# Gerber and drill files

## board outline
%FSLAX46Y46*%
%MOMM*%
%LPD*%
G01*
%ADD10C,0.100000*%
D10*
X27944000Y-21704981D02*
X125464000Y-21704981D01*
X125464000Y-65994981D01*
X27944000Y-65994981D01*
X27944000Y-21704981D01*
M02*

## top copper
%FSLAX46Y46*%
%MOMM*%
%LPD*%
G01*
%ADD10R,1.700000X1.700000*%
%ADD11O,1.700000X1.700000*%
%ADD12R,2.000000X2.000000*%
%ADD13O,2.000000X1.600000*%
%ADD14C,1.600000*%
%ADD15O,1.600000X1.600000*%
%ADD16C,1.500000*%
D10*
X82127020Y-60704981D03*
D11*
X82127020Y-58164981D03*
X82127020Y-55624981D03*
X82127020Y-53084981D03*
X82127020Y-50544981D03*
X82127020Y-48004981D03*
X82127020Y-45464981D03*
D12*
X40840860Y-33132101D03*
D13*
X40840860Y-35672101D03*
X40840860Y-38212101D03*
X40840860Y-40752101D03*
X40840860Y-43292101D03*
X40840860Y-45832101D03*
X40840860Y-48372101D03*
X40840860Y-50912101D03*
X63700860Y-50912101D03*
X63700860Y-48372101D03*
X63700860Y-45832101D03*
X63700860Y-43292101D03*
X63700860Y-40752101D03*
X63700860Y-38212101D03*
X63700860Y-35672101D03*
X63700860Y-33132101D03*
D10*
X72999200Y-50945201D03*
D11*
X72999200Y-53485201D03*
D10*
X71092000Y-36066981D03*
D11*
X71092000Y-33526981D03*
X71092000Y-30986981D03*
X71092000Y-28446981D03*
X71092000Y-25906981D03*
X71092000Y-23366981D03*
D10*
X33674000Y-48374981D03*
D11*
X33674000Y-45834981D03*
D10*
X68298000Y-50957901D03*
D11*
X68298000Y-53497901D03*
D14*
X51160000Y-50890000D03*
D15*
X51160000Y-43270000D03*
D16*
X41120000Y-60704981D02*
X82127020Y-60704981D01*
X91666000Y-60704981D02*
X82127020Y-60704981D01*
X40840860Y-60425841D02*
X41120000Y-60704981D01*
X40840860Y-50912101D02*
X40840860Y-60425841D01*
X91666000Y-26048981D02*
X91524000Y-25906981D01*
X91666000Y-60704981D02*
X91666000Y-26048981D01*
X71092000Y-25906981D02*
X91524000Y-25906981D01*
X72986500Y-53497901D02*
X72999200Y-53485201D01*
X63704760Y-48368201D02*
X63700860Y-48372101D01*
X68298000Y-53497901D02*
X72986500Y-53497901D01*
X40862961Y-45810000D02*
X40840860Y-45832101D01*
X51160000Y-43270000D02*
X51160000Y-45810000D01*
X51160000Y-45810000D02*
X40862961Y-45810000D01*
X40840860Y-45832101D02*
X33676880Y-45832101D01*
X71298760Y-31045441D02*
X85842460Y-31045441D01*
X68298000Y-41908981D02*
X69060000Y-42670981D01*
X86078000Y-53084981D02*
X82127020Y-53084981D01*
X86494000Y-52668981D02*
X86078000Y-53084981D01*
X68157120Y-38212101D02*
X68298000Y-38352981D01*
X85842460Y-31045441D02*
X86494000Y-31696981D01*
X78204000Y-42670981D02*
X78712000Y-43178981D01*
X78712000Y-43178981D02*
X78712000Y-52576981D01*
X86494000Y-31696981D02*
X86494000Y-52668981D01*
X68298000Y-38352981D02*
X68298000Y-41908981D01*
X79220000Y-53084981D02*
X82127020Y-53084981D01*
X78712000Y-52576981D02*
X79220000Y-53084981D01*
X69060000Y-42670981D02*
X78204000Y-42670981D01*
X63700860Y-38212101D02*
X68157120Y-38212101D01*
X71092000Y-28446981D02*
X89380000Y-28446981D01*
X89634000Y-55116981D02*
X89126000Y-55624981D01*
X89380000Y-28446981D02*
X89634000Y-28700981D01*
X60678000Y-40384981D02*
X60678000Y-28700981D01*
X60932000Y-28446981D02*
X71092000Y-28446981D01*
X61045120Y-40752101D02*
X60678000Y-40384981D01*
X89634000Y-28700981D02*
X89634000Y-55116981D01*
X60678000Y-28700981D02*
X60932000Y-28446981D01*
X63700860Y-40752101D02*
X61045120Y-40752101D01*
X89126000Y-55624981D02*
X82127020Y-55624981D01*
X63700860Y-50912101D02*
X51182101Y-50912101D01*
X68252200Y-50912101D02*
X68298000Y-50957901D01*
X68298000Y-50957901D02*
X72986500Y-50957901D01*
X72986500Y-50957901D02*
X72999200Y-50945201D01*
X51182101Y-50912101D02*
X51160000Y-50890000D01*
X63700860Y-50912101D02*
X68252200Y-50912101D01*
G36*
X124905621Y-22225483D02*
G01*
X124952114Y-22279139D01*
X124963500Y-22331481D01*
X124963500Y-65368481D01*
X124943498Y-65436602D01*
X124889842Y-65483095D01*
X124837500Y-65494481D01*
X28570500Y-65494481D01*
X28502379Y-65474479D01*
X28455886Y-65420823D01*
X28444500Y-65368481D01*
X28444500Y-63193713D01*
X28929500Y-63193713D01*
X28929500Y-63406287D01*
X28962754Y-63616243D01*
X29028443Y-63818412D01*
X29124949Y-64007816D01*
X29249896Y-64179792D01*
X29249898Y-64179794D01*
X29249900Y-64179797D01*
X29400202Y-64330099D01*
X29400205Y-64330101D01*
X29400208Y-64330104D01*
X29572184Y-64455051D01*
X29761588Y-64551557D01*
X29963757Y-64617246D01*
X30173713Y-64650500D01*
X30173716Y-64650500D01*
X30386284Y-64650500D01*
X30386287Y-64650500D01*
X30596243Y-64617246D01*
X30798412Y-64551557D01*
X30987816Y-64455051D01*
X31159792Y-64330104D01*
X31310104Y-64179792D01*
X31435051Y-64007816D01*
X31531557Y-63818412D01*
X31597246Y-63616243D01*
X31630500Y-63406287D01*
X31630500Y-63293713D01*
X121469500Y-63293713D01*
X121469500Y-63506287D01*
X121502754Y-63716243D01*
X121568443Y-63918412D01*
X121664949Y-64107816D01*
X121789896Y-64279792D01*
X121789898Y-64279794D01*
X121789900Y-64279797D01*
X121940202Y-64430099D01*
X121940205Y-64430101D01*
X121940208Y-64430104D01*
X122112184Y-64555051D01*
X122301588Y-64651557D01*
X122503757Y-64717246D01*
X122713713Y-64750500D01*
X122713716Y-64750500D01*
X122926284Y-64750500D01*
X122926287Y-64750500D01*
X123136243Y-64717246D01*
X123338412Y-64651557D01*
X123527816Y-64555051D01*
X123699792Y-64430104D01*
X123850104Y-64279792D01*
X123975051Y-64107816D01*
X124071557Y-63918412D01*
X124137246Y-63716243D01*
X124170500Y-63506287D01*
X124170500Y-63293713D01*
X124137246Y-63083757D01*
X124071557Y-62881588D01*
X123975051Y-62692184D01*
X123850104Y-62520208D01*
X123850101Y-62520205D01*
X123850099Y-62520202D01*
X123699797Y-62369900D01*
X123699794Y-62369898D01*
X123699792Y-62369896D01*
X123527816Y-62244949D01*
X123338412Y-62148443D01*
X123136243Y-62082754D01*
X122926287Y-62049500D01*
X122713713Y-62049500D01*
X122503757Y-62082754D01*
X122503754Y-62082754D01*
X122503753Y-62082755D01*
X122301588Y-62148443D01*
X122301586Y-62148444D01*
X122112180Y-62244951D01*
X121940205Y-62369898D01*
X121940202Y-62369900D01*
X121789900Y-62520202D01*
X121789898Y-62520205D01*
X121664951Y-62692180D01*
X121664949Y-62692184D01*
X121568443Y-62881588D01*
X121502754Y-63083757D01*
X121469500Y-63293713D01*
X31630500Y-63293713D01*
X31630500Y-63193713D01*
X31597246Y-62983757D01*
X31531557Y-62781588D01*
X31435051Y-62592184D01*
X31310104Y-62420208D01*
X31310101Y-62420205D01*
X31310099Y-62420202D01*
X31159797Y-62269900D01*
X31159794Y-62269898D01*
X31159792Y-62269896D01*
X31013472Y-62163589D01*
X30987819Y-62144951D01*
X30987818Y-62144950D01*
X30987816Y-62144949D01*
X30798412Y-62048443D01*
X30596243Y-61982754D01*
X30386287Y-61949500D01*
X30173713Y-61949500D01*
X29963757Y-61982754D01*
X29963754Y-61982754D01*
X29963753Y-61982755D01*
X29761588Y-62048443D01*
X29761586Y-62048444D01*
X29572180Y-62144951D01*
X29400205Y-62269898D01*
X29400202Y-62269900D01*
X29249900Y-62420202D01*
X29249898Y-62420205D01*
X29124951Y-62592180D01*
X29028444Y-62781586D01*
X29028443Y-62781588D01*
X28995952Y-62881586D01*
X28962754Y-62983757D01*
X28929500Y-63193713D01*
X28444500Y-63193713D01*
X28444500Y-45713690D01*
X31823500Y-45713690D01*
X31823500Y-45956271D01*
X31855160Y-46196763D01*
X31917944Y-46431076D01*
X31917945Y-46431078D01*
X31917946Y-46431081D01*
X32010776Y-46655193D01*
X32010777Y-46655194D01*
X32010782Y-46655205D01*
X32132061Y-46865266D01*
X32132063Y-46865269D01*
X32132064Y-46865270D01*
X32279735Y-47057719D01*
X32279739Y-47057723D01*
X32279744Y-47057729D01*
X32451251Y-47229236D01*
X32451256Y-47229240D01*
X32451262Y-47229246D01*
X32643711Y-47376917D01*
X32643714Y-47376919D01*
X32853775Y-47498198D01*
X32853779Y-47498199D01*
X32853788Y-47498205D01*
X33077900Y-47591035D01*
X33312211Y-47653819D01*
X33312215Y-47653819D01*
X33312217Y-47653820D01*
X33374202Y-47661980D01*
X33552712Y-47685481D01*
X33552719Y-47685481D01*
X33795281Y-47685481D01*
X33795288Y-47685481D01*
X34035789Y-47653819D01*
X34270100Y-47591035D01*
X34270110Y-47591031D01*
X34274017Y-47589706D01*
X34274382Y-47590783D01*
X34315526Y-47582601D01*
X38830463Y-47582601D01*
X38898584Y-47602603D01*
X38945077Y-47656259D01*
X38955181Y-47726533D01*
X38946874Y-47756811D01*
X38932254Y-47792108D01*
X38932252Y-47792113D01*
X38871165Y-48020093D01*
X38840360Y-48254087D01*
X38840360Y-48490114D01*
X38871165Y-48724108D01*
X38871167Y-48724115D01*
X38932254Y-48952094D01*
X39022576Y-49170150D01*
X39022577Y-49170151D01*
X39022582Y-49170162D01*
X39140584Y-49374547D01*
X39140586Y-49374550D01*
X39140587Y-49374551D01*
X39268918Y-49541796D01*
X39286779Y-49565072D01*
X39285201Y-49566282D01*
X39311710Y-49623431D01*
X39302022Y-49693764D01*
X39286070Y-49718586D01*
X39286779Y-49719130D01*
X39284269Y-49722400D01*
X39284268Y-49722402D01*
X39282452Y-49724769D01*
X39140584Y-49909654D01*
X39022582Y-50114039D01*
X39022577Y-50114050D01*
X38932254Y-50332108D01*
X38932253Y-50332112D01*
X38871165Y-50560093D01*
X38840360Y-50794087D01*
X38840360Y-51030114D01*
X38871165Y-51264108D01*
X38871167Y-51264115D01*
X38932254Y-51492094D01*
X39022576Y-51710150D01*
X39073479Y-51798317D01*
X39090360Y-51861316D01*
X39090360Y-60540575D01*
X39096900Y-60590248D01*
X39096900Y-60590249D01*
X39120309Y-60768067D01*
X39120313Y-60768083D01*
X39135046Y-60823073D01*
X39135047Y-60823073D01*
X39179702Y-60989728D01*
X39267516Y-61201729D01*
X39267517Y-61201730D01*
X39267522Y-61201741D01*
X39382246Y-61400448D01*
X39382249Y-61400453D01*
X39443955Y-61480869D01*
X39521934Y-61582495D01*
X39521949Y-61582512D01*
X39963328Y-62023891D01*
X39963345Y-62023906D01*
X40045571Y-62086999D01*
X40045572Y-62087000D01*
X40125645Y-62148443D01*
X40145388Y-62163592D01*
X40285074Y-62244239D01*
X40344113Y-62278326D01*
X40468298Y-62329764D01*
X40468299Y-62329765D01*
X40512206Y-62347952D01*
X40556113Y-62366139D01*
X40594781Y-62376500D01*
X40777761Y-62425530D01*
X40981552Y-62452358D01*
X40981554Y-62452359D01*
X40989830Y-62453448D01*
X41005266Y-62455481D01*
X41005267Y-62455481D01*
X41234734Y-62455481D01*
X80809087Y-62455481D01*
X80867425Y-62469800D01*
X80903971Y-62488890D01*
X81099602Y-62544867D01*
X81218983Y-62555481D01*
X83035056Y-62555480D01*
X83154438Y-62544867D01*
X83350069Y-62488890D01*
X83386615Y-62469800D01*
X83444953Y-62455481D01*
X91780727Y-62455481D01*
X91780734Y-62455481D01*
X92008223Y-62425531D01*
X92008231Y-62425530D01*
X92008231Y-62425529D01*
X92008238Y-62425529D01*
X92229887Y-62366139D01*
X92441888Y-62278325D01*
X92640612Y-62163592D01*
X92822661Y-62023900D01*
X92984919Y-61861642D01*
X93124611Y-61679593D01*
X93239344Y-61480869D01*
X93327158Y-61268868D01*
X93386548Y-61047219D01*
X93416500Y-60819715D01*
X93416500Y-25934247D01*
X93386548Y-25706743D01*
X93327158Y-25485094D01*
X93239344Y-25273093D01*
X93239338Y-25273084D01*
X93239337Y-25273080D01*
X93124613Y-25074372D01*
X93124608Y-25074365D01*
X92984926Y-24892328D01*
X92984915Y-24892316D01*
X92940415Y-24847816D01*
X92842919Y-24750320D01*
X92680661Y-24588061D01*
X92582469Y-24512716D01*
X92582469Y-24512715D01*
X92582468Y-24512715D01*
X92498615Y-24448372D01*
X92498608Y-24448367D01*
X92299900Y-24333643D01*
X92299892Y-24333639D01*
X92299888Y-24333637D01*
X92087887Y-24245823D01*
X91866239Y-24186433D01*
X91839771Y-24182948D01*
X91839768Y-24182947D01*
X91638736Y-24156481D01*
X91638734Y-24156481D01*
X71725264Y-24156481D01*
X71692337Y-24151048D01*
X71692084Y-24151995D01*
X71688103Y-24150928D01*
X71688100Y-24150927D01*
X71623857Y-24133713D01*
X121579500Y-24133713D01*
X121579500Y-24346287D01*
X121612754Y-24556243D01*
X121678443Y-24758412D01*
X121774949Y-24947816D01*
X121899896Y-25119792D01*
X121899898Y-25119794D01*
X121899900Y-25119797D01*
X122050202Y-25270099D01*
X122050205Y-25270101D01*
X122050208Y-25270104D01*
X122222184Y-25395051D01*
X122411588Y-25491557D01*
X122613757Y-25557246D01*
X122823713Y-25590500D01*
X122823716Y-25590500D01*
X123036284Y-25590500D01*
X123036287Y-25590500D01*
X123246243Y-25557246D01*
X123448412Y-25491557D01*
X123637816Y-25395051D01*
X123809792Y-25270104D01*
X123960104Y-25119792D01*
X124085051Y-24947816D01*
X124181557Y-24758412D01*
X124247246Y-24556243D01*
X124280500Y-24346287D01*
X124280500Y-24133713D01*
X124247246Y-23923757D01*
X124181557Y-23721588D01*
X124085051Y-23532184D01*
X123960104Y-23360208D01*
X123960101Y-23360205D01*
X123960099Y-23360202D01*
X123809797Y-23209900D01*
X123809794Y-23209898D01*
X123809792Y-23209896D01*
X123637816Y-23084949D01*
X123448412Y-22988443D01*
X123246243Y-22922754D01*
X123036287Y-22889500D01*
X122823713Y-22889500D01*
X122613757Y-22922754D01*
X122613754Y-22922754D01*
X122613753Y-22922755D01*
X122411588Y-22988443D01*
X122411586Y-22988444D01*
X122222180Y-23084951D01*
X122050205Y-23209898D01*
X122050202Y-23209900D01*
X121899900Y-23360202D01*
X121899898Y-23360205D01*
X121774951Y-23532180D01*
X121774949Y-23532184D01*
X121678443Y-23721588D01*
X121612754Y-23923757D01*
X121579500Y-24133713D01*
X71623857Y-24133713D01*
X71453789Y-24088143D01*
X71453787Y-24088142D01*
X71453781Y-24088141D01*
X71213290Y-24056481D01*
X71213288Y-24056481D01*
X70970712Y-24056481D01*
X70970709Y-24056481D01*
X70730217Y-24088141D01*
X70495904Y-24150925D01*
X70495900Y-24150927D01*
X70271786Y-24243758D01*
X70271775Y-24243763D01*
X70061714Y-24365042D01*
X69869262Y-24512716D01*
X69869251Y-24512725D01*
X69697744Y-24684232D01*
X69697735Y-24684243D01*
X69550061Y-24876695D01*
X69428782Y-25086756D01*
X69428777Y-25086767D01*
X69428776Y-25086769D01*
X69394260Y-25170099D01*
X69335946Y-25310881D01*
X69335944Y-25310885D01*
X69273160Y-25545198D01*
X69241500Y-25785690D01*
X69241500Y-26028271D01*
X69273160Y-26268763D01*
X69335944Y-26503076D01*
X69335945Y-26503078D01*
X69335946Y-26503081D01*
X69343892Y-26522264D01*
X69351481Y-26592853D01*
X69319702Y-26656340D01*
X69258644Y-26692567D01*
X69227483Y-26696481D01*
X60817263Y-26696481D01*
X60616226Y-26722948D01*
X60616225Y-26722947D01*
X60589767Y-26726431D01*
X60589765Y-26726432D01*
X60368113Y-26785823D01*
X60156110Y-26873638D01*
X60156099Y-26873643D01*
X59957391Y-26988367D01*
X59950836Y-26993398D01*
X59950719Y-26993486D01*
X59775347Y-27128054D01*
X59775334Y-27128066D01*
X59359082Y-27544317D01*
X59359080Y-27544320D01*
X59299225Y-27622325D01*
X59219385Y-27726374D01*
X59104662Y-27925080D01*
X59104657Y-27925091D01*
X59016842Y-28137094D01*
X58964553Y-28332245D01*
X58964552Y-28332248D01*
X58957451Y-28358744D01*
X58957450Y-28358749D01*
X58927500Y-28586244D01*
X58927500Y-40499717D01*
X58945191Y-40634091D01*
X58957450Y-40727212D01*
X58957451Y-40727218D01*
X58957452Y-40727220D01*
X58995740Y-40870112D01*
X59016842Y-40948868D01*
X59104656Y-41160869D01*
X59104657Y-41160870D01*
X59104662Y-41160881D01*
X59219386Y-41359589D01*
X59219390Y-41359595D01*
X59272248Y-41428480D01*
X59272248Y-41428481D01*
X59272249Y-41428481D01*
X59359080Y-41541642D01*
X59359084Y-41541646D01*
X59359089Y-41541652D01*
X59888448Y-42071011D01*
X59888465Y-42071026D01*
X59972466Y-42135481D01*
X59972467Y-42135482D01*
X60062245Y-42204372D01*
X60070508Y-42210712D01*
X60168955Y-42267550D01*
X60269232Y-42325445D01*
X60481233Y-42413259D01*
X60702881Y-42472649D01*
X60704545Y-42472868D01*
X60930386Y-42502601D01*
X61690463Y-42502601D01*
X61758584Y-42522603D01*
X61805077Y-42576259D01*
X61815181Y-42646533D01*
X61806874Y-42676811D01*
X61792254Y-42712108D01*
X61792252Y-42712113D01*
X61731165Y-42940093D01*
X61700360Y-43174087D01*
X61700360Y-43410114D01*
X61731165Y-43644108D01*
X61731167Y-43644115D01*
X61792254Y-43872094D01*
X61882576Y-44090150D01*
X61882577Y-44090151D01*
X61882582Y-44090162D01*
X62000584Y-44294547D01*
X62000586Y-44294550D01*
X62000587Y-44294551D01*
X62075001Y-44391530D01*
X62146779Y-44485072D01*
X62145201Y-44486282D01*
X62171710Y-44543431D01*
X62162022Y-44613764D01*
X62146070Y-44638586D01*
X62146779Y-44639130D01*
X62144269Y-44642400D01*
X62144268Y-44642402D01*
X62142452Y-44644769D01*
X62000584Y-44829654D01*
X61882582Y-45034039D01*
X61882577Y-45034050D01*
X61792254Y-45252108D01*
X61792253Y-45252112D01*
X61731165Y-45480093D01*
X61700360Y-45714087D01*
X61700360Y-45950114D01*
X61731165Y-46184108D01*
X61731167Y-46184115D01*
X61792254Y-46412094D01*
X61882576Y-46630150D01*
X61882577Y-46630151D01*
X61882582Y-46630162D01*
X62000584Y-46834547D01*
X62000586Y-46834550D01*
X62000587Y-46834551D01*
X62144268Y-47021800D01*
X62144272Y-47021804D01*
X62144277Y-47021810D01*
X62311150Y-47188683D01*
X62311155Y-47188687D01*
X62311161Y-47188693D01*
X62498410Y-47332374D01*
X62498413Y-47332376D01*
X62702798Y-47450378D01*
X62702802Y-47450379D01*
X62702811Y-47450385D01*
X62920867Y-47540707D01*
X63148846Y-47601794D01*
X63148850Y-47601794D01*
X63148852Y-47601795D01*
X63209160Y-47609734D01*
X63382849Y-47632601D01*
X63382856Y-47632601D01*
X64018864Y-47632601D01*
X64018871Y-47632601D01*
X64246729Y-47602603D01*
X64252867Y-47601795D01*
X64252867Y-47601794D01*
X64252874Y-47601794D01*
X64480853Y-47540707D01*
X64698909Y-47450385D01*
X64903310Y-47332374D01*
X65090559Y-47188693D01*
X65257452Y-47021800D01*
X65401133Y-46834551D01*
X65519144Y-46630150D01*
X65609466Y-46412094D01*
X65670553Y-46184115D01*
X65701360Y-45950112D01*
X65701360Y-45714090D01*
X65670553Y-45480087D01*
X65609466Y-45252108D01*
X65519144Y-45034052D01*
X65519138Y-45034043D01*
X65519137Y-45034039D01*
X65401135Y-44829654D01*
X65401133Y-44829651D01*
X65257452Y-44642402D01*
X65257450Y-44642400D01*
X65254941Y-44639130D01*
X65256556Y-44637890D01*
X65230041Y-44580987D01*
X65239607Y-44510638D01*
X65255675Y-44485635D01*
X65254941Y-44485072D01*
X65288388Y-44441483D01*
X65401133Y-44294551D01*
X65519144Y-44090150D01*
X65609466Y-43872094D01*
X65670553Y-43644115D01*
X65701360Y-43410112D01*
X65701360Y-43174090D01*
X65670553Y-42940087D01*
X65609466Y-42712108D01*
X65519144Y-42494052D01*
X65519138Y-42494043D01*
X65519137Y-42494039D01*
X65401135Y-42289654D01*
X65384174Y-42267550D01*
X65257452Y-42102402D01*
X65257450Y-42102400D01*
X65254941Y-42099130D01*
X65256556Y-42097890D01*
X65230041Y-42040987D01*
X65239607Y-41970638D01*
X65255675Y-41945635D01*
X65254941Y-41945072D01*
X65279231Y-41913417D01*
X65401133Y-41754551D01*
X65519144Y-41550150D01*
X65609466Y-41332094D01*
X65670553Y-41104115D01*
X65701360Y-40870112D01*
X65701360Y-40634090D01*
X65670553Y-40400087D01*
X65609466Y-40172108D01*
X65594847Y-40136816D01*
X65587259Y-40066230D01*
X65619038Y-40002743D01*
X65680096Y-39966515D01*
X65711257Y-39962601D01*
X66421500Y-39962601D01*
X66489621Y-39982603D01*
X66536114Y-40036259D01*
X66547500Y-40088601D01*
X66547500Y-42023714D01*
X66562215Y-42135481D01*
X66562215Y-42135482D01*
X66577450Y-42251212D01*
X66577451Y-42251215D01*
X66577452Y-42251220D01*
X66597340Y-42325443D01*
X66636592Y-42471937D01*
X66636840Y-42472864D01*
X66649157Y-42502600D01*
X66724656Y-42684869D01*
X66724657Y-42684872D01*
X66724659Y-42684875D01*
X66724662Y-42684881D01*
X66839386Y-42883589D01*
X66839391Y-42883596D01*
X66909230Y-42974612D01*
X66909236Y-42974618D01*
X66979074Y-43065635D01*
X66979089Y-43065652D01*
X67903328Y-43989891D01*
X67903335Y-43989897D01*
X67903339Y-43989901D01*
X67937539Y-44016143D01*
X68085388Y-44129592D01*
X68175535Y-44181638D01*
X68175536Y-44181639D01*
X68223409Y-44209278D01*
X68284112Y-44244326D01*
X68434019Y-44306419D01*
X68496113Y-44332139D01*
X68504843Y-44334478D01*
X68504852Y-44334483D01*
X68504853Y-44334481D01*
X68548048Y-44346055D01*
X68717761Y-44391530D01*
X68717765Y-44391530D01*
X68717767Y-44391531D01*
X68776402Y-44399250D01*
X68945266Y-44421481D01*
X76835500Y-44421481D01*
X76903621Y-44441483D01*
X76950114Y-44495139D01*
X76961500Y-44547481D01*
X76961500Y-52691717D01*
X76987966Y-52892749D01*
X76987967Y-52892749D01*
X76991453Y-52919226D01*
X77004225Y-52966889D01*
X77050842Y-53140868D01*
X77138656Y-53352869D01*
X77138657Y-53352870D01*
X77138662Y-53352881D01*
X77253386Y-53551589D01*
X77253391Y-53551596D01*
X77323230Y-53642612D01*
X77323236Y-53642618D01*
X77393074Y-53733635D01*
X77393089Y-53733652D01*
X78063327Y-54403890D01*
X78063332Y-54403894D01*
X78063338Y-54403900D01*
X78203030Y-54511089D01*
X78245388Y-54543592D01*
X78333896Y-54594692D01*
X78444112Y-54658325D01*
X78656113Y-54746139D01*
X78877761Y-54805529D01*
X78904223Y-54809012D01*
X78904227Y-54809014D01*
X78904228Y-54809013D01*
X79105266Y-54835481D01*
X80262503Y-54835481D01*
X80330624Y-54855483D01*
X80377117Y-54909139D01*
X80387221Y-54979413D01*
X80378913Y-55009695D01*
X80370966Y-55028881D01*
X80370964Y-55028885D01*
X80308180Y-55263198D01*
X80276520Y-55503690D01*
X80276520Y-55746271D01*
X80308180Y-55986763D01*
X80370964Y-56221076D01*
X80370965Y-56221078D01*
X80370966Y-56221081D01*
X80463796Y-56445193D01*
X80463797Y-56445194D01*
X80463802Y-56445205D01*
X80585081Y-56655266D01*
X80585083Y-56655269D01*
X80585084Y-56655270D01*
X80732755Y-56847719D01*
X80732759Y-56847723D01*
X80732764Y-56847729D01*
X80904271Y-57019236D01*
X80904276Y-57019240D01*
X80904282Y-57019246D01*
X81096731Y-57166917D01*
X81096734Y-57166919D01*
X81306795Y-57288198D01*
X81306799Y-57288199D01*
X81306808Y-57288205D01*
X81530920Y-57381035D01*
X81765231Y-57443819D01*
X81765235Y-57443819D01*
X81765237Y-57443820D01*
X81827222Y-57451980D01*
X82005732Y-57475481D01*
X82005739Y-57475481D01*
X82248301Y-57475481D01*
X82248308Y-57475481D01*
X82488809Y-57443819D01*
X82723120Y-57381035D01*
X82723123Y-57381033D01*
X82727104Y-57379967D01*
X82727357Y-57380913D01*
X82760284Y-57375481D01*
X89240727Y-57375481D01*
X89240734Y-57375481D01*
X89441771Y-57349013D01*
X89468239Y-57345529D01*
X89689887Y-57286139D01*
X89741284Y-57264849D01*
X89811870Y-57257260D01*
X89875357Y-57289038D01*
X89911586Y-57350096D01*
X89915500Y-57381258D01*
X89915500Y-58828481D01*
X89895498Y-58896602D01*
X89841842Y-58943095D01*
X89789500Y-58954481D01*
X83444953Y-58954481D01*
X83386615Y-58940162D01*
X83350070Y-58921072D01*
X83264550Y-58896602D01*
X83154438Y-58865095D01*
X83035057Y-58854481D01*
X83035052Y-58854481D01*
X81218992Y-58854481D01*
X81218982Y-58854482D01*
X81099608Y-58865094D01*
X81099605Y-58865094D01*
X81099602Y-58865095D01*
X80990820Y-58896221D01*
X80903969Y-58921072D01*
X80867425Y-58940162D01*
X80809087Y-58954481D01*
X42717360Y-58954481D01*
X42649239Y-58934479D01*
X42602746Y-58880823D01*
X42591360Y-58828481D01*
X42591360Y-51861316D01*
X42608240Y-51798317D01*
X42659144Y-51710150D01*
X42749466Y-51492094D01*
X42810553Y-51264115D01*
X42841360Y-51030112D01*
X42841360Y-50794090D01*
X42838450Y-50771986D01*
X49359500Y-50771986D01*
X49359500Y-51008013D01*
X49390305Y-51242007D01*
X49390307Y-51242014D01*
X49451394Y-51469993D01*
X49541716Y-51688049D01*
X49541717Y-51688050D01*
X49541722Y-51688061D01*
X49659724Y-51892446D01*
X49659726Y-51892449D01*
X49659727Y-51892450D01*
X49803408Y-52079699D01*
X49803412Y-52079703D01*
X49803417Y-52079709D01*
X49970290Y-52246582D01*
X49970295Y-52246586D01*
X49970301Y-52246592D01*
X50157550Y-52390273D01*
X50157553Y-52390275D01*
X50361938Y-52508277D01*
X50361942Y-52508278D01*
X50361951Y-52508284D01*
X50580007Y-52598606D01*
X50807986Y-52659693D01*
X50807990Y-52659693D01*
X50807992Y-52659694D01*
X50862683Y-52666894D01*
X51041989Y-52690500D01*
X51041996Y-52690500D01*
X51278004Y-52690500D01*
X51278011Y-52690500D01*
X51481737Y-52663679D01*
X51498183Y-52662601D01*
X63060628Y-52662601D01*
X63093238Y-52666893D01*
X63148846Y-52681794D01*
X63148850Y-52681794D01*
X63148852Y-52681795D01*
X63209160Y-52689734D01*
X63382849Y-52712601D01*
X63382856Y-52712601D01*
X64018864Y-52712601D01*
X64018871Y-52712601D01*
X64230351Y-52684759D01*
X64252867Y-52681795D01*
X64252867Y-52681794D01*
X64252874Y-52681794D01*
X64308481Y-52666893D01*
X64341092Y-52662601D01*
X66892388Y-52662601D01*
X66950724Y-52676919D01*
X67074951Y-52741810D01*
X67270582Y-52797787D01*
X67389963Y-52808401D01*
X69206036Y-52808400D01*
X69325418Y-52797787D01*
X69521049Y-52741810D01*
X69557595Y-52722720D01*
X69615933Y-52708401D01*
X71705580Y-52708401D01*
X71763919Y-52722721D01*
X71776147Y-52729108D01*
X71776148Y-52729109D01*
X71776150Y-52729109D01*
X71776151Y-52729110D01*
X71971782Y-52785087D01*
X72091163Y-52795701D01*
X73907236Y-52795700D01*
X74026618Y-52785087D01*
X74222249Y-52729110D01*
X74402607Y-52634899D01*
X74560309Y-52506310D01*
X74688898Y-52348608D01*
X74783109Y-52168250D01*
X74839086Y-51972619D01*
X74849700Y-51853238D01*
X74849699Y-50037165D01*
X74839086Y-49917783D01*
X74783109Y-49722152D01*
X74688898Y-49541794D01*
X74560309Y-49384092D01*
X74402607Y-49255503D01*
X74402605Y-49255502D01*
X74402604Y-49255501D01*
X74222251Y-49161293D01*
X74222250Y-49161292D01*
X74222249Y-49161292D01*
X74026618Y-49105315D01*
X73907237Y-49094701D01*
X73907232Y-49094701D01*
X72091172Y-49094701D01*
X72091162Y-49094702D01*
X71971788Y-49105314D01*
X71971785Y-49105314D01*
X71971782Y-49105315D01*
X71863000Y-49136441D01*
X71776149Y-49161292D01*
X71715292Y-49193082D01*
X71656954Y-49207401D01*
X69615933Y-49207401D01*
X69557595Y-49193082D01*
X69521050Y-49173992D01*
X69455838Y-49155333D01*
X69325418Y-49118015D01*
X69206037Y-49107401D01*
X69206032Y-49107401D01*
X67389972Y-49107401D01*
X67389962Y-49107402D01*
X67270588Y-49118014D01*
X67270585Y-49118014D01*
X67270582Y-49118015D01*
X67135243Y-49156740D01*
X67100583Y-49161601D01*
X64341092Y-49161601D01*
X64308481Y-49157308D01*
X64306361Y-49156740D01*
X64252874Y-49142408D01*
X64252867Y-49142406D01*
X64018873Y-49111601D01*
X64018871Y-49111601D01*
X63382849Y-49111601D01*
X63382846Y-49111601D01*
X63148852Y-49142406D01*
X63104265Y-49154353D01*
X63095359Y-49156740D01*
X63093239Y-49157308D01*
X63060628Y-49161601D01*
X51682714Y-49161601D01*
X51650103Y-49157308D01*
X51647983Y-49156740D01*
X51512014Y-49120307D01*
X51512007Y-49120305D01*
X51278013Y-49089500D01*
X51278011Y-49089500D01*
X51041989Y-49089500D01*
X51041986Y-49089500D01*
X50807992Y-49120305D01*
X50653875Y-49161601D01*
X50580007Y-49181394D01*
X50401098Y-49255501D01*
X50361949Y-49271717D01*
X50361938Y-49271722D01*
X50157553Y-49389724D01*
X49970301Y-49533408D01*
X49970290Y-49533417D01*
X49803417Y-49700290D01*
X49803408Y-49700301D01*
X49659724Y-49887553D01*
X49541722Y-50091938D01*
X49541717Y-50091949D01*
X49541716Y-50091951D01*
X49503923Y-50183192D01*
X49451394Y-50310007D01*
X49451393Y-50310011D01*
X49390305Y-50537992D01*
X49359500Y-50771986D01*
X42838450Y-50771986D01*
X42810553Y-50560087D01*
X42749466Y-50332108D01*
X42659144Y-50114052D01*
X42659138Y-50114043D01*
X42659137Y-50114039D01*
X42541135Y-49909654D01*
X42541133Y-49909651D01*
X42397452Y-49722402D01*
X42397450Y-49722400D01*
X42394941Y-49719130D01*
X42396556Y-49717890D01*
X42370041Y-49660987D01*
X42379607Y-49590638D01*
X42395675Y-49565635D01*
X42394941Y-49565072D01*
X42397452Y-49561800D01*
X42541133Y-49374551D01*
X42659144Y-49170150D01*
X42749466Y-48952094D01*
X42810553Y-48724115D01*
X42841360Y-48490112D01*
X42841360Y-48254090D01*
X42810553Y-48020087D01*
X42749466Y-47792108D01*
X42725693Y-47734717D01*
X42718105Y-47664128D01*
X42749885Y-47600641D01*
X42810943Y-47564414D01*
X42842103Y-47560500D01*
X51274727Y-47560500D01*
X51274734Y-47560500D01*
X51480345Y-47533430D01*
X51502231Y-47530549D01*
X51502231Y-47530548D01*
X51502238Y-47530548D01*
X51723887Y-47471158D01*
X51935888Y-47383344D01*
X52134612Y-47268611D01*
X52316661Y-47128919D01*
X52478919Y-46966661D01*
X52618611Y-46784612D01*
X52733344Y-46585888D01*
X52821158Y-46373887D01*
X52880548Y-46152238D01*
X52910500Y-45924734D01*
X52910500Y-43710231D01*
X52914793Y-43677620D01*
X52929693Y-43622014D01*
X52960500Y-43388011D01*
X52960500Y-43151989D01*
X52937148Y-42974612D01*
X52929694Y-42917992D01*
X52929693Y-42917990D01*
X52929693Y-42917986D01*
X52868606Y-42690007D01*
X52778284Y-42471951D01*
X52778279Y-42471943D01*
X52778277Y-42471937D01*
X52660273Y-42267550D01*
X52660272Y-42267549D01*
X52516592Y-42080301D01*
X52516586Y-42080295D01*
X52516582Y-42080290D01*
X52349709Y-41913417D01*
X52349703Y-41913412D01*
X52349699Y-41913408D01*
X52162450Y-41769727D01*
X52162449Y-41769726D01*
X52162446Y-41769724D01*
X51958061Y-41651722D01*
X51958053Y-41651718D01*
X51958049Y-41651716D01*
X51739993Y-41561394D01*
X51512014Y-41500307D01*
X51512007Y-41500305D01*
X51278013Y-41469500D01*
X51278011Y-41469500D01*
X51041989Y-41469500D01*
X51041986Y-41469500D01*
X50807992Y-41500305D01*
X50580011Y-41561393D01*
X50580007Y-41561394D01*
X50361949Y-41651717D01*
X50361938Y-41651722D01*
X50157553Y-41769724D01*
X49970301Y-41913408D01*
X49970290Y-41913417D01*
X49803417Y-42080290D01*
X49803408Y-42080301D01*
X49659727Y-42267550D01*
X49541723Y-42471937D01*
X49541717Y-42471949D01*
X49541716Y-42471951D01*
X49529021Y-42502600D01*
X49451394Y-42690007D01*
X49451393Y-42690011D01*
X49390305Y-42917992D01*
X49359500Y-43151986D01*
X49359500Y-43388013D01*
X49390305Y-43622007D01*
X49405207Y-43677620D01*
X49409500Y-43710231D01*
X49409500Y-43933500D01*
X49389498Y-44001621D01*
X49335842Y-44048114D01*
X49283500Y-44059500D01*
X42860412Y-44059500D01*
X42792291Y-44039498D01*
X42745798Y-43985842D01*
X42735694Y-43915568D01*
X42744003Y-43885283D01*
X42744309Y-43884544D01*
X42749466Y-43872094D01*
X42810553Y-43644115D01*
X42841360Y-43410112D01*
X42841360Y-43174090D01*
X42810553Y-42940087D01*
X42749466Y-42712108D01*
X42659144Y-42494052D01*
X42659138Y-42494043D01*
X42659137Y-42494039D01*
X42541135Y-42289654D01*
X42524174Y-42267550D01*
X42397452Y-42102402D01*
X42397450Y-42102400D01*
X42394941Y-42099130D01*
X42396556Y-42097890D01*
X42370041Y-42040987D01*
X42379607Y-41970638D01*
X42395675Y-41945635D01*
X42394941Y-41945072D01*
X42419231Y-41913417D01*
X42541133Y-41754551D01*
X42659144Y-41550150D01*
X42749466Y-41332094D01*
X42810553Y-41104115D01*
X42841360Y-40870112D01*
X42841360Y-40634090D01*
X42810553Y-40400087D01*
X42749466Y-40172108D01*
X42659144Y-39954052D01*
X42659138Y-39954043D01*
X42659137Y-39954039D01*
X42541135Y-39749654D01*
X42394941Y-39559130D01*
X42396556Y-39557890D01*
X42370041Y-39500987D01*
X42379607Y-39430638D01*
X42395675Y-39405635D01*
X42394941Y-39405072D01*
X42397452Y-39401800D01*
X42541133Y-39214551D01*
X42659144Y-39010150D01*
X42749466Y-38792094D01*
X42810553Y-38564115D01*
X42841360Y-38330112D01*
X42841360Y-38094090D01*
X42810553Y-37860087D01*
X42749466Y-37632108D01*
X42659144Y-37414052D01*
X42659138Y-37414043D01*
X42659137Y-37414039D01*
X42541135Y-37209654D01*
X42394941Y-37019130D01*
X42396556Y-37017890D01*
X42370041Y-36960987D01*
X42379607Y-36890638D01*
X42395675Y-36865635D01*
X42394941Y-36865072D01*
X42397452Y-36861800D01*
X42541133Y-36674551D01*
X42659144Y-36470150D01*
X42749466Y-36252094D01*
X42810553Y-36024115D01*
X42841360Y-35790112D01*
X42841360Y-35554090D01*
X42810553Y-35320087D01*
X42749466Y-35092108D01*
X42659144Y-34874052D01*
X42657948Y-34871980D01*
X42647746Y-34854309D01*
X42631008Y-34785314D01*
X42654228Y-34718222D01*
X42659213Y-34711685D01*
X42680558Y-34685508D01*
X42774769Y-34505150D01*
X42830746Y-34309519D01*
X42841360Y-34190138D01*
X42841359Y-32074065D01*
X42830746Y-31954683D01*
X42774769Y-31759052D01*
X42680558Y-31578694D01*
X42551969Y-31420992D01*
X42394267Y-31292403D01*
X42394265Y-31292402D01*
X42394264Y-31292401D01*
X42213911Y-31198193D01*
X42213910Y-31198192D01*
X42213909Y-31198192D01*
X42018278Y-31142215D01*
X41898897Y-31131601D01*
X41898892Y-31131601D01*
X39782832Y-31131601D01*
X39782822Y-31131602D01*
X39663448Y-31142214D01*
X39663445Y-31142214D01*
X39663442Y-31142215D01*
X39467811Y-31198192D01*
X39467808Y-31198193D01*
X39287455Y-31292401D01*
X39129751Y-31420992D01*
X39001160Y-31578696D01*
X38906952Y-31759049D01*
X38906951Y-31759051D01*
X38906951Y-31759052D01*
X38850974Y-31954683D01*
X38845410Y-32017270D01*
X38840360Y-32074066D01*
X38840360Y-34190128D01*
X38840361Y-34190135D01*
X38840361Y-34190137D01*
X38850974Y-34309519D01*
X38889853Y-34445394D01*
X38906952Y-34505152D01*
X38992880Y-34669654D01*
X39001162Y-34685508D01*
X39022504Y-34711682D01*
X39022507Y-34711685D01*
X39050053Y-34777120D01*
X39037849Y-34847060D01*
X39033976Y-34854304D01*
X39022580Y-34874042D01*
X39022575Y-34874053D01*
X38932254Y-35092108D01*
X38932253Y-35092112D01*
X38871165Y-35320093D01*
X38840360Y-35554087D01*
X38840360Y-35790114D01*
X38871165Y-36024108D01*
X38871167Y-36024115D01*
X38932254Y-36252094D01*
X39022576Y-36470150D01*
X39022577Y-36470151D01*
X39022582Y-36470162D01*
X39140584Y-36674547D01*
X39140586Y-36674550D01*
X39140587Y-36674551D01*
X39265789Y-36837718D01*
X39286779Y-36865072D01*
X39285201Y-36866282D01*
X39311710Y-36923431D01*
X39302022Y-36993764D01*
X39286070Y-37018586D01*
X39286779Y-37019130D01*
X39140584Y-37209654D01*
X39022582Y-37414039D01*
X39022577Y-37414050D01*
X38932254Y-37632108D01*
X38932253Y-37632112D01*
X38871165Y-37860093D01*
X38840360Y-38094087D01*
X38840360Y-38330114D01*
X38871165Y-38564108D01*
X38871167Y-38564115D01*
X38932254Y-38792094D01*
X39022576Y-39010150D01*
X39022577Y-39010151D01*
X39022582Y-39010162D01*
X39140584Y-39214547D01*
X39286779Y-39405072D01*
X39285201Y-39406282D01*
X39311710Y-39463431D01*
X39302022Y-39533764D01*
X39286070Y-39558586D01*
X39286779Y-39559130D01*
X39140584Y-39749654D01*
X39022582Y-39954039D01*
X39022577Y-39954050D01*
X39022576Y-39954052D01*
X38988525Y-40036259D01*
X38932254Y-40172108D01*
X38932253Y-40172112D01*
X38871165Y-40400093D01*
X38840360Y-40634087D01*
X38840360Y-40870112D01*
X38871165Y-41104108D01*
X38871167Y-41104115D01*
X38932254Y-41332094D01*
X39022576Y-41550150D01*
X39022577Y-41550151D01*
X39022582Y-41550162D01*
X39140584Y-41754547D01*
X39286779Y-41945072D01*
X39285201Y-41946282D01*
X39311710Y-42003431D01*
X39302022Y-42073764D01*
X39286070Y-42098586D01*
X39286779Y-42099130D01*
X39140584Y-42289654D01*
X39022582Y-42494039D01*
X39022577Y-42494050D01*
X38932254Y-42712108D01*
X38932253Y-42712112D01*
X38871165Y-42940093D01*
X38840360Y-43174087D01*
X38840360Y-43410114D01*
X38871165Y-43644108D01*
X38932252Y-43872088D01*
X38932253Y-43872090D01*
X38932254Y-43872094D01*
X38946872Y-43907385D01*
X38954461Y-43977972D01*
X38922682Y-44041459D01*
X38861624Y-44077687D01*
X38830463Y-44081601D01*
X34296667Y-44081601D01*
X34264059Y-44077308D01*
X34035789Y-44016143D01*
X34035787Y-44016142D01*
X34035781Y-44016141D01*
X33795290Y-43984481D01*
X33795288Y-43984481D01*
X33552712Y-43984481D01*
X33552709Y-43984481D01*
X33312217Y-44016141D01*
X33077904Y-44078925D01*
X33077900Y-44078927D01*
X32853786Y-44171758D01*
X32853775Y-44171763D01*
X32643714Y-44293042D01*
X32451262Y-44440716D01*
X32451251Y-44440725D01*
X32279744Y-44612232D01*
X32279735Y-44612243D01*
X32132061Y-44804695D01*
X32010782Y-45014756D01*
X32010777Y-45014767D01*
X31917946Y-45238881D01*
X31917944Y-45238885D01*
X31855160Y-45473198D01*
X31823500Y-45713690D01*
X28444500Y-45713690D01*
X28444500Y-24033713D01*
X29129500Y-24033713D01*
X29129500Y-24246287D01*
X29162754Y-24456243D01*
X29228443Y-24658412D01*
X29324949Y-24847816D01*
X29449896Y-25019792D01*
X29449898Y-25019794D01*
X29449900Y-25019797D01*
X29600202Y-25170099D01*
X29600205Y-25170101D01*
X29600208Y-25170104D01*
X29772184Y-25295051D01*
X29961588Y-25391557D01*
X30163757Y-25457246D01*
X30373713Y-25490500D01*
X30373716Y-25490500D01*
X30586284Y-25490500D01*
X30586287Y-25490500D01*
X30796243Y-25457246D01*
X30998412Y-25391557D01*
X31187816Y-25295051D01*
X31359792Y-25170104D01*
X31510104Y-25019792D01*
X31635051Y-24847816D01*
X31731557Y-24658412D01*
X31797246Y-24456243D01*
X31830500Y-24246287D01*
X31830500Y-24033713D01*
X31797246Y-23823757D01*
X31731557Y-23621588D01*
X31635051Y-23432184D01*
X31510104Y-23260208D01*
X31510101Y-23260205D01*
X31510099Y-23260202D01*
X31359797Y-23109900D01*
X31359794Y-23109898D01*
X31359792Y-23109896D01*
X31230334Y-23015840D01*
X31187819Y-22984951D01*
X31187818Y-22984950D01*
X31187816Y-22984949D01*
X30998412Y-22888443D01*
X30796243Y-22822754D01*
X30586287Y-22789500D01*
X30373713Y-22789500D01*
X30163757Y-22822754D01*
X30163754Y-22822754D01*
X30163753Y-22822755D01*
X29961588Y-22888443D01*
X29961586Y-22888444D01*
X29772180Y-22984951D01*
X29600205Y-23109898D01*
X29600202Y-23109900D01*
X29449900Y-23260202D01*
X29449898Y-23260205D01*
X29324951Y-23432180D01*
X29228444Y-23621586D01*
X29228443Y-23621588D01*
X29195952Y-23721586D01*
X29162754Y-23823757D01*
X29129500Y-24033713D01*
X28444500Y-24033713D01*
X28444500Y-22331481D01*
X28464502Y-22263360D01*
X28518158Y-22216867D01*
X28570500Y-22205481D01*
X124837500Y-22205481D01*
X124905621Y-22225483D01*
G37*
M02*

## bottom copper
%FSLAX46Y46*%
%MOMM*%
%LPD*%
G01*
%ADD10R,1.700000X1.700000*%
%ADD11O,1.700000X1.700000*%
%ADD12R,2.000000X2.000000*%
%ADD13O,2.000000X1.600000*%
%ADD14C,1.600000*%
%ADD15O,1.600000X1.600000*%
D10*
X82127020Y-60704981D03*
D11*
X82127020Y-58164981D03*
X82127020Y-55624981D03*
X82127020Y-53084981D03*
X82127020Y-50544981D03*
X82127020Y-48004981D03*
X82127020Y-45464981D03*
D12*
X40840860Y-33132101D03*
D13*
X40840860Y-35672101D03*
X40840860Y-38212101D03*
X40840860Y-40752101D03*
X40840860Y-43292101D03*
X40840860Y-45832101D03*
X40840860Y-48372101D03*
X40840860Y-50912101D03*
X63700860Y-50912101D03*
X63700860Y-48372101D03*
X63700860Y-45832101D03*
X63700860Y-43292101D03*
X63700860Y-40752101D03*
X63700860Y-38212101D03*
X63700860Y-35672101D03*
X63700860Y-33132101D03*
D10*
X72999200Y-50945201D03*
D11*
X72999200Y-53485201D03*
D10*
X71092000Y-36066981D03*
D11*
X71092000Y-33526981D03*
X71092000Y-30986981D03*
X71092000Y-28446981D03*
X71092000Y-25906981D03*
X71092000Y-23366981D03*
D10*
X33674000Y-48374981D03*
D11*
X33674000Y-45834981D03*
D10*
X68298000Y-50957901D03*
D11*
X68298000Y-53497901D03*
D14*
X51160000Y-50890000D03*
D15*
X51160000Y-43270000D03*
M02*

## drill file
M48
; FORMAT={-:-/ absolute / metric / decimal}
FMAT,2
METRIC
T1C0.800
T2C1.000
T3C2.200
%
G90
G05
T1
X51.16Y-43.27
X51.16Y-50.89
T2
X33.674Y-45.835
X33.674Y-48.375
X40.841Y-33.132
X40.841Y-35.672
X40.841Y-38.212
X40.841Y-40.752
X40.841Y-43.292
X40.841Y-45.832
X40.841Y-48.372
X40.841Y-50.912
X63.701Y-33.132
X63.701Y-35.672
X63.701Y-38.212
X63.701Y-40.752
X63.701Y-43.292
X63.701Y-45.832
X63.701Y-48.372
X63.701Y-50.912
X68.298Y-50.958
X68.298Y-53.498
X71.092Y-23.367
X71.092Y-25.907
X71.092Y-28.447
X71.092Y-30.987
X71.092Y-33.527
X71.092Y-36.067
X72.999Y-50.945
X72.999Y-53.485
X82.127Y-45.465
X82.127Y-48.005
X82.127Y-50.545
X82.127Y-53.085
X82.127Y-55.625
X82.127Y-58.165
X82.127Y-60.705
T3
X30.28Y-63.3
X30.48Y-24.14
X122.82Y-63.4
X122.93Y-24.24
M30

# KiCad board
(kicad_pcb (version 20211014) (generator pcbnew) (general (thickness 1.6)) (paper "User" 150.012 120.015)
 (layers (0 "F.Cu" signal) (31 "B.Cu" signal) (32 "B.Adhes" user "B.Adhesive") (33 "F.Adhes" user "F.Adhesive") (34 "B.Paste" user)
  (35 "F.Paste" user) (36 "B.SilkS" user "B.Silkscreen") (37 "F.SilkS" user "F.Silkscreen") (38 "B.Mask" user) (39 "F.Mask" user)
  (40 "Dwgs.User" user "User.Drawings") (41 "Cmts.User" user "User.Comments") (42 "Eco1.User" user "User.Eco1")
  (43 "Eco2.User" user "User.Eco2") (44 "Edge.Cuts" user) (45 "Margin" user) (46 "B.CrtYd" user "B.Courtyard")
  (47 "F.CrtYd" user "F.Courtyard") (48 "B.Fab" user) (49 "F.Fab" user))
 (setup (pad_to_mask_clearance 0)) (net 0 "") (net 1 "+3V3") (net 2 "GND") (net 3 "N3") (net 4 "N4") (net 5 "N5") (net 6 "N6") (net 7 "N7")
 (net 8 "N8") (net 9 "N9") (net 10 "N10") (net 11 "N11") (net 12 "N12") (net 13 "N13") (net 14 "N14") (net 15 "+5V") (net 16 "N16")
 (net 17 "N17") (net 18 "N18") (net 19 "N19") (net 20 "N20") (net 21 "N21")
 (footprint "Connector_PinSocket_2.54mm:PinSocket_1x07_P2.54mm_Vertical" (layer "F.Cu") (at 82.12702 60.704981 180)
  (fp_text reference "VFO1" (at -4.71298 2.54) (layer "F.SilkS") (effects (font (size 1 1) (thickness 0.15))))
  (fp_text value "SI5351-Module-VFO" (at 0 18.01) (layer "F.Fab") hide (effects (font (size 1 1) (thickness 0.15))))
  (pad "1" thru_hole rect locked (at 0 0 180) (size 1.7 1.7) (drill 1) (layers *.Cu *.Mask) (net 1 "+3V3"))
  (pad "2" thru_hole oval locked (at 0 2.54 180) (size 1.7 1.7) (drill 1) (layers *.Cu *.Mask) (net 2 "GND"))
  (pad "3" thru_hole oval locked (at 0 5.08 180) (size 1.7 1.7) (drill 1) (layers *.Cu *.Mask) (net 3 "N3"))
  (pad "4" thru_hole oval locked (at 0 7.62 180) (size 1.7 1.7) (drill 1) (layers *.Cu *.Mask) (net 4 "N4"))
  (pad "5" thru_hole oval locked (at 0 10.16 180) (size 1.7 1.7) (drill 1) (layers *.Cu *.Mask) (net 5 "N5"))
  (pad "6" thru_hole oval locked (at 0 12.7 180) (size 1.7 1.7) (drill 1) (layers *.Cu *.Mask) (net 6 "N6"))
  (pad "7" thru_hole oval locked (at 0 15.24 180) (size 1.7 1.7) (drill 1) (layers *.Cu *.Mask) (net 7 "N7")))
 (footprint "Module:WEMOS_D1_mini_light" (layer "F.Cu") (at 40.84086 33.132101)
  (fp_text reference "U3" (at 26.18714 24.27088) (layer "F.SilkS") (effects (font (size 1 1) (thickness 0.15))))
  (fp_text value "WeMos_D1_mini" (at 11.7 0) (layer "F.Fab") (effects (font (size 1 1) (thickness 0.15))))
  (pad "1" thru_hole rect (at 0 0) (size 2 2) (drill 1) (layers *.Cu *.Mask) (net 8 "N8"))
  (pad "2" thru_hole oval (at 0 2.54) (size 2 1.6) (drill 1) (layers *.Cu *.Mask) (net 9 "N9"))
  (pad "3" thru_hole oval (at 0 5.08) (size 2 1.6) (drill 1) (layers *.Cu *.Mask) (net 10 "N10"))
  (pad "4" thru_hole oval (at 0 7.62) (size 2 1.6) (drill 1) (layers *.Cu *.Mask) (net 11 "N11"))
  (pad "5" thru_hole oval (at 0 10.16) (size 2 1.6) (drill 1) (layers *.Cu *.Mask) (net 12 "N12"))
  (pad "6" thru_hole oval (at 0 12.7) (size 2 1.6) (drill 1) (layers *.Cu *.Mask) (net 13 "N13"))
  (pad "7" thru_hole oval (at 0 15.24) (size 2 1.6) (drill 1) (layers *.Cu *.Mask) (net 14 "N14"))
  (pad "8" thru_hole oval (at 0 17.78) (size 2 1.6) (drill 1) (layers *.Cu *.Mask) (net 1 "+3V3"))
  (pad "9" thru_hole oval (at 22.86 17.78) (size 2 1.6) (drill 1) (layers *.Cu *.Mask) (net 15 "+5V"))
  (pad "10" thru_hole oval (at 22.86 15.24) (size 2 1.6) (drill 1) (layers *.Cu *.Mask) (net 2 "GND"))
  (pad "11" thru_hole oval (at 22.86 12.7) (size 2 1.6) (drill 1) (layers *.Cu *.Mask) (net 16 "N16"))
  (pad "12" thru_hole oval (at 22.86 10.16) (size 2 1.6) (drill 1) (layers *.Cu *.Mask) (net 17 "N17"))
  (pad "13" thru_hole oval (at 22.86 7.62) (size 2 1.6) (drill 1) (layers *.Cu *.Mask) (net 3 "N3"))
  (pad "14" thru_hole oval (at 22.86 5.08) (size 2 1.6) (drill 1) (layers *.Cu *.Mask) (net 4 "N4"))
  (pad "15" thru_hole oval (at 22.86 2.54) (size 2 1.6) (drill 1) (layers *.Cu *.Mask) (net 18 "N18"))
  (pad "16" thru_hole oval (at 22.86 0) (size 2 1.6) (drill 1) (layers *.Cu *.Mask) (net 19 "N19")))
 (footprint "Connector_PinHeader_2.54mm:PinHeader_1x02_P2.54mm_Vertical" (layer "F.Cu") (at 72.9992 50.945201)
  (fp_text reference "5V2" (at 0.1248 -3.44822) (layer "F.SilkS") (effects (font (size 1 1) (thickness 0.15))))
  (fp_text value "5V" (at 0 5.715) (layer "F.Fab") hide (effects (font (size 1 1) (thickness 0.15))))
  (pad "1" thru_hole rect locked (at 0 0) (size 1.7 1.7) (drill 1) (layers *.Cu *.Mask) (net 15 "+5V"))
  (pad "2" thru_hole oval locked (at 0 2.54) (size 1.7 1.7) (drill 1) (layers *.Cu *.Mask) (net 2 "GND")))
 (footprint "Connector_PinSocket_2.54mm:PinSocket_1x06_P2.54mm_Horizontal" (layer "F.Cu") (at 71.092 36.066981 180)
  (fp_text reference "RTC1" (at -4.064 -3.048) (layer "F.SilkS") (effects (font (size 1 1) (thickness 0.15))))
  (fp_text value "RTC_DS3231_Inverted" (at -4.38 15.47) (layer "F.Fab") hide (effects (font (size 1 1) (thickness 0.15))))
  (pad "1" thru_hole rect locked (at 0 0 180) (size 1.7 1.7) (drill 1) (layers *.Cu *.Mask) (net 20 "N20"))
  (pad "2" thru_hole oval locked (at 0 2.54 180) (size 1.7 1.7) (drill 1) (layers *.Cu *.Mask) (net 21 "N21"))
  (pad "3" thru_hole oval locked (at 0 5.08 180) (size 1.7 1.7) (drill 1) (layers *.Cu *.Mask) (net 4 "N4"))
  (pad "4" thru_hole oval locked (at 0 7.62 180) (size 1.7 1.7) (drill 1) (layers *.Cu *.Mask) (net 3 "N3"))
  (pad "5" thru_hole oval locked (at 0 10.16 180) (size 1.7 1.7) (drill 1) (layers *.Cu *.Mask) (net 1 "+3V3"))
  (pad "6" thru_hole oval locked (at 0 12.7 180) (size 1.7 1.7) (drill 1) (layers *.Cu *.Mask) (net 2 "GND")))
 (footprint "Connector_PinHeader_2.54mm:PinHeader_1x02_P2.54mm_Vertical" (layer "F.Cu") (at 33.674 48.374981 180)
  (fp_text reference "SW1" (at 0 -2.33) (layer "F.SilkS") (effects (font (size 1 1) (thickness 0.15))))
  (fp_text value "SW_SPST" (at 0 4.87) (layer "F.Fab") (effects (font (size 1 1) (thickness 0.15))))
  (pad "1" thru_hole rect locked (at 0 0 180) (size 1.7 1.7) (drill 1) (layers *.Cu *.Mask) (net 2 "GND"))
  (pad "2" thru_hole oval locked (at 0 2.54 180) (size 1.7 1.7) (drill 1) (layers *.Cu *.Mask) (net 13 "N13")))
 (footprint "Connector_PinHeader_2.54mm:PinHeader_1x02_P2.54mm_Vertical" (layer "F.Cu") (at 68.298 50.957901)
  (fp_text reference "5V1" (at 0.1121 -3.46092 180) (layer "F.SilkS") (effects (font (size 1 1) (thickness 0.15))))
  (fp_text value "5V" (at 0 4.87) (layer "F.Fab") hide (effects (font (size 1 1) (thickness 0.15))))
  (pad "1" thru_hole rect locked (at 0 0) (size 1.7 1.7) (drill 1) (layers *.Cu *.Mask) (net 15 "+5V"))
  (pad "2" thru_hole oval locked (at 0 2.54) (size 1.7 1.7) (drill 1) (layers *.Cu *.Mask) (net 2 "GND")))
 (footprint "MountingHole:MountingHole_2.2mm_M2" (layer "F.Cu") (at 122.93 24.24)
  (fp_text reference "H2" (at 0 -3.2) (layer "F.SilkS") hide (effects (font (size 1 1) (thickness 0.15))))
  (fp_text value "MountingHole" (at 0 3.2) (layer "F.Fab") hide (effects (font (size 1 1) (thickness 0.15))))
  (pad "" np_thru_hole circle (at 0 0) (size 2.2 2.2) (drill 2.2) (layers *.Cu *.Mask)))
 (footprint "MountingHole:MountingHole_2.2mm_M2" (layer "F.Cu") (at 30.28 63.3)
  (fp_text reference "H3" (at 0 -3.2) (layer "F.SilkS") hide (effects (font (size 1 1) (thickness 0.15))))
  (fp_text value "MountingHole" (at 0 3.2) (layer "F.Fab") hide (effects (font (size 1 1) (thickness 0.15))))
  (pad "" np_thru_hole circle (at 0 0) (size 2.2 2.2) (drill 2.2) (layers *.Cu *.Mask)))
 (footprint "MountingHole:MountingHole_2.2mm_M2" (layer "F.Cu") (at 30.48 24.14)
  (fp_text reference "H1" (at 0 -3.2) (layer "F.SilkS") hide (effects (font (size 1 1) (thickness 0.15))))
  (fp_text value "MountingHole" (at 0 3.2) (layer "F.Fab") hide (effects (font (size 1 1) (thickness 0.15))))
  (pad "" np_thru_hole circle (at 0 0) (size 2.2 2.2) (drill 2.2) (layers *.Cu *.Mask)))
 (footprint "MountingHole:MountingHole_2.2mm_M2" (layer "F.Cu") (at 122.82 63.4)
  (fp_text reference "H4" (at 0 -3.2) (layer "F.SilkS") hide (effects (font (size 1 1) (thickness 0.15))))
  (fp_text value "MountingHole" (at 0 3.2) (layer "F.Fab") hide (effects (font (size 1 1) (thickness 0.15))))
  (pad "" np_thru_hole circle (at 0 0) (size 2.2 2.2) (drill 2.2) (layers *.Cu *.Mask)))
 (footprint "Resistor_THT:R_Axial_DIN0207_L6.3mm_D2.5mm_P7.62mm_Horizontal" (layer "B.Cu") (at 51.16 50.89 90)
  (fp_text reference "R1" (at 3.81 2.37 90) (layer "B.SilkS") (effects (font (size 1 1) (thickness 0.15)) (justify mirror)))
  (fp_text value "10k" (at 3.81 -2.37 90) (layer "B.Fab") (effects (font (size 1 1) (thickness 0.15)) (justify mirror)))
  (pad "1" thru_hole circle (at 0 0 90) (size 1.6 1.6) (drill 0.8) (layers *.Cu *.Mask) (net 15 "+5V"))
  (pad "2" thru_hole oval (at 7.62 0 90) (size 1.6 1.6) (drill 0.8) (layers *.Cu *.Mask) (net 13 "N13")))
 (gr_rect (start 27.944 21.704981) (end 125.464 65.994981) (layer "Edge.Cuts") (width 0.1) (fill none))
 (segment (start 41.12 60.704981) (end 82.12702 60.704981) (width 1.5) (layer "F.Cu") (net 1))
 (segment (start 91.666 60.704981) (end 82.12702 60.704981) (width 1.5) (layer "F.Cu") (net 1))
 (segment (start 40.84086 60.425841) (end 41.12 60.704981) (width 1.5) (layer "F.Cu") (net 1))
 (segment (start 40.84086 50.912101) (end 40.84086 60.425841) (width 1.5) (layer "F.Cu") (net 1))
 (segment (start 91.666 26.048981) (end 91.524 25.906981) (width 1.5) (layer "F.Cu") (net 1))
 (segment (start 91.666 60.704981) (end 91.666 26.048981) (width 1.5) (layer "F.Cu") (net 1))
 (segment (start 71.092 25.906981) (end 91.524 25.906981) (width 1.5) (layer "F.Cu") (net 1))
 (segment (start 72.9865 53.497901) (end 72.9992 53.485201) (width 1.5) (layer "F.Cu") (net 2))
 (segment (start 63.70476 48.368201) (end 63.70086 48.372101) (width 1.5) (layer "F.Cu") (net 2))
 (segment (start 68.298 53.497901) (end 72.9865 53.497901) (width 1.5) (layer "F.Cu") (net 2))
 (segment (start 40.862961 45.81) (end 40.84086 45.832101) (width 1.5) (layer "F.Cu") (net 13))
 (segment (start 51.16 43.27) (end 51.16 45.81) (width 1.5) (layer "F.Cu") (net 13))
 (segment (start 51.16 45.81) (end 40.862961 45.81) (width 1.5) (layer "F.Cu") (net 13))
 (segment (start 40.84086 45.832101) (end 33.67688 45.832101) (width 1.5) (layer "F.Cu") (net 13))
 (segment (start 71.29876 31.045441) (end 85.84246 31.045441) (width 1.5) (layer "F.Cu") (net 4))
 (segment (start 68.298 41.908981) (end 69.06 42.670981) (width 1.5) (layer "F.Cu") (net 4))
 (segment (start 86.078 53.084981) (end 82.12702 53.084981) (width 1.5) (layer "F.Cu") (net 4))
 (segment (start 86.494 52.668981) (end 86.078 53.084981) (width 1.5) (layer "F.Cu") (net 4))
 (segment (start 68.15712 38.212101) (end 68.298 38.352981) (width 1.5) (layer "F.Cu") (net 4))
 (segment (start 85.84246 31.045441) (end 86.494 31.696981) (width 1.5) (layer "F.Cu") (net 4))
 (segment (start 78.204 42.670981) (end 78.712 43.178981) (width 1.5) (layer "F.Cu") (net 4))
 (segment (start 78.712 43.178981) (end 78.712 52.576981) (width 1.5) (layer "F.Cu") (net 4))
 (segment (start 86.494 31.696981) (end 86.494 52.668981) (width 1.5) (layer "F.Cu") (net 4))
 (segment (start 68.298 38.352981) (end 68.298 41.908981) (width 1.5) (layer "F.Cu") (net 4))
 (segment (start 79.22 53.084981) (end 82.12702 53.084981) (width 1.5) (layer "F.Cu") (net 4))
 (segment (start 78.712 52.576981) (end 79.22 53.084981) (width 1.5) (layer "F.Cu") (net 4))
 (segment (start 69.06 42.670981) (end 78.204 42.670981) (width 1.5) (layer "F.Cu") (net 4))
 (segment (start 63.70086 38.212101) (end 68.15712 38.212101) (width 1.5) (layer "F.Cu") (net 4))
 (segment (start 71.092 28.446981) (end 89.38 28.446981) (width 1.5) (layer "F.Cu") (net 3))
 (segment (start 89.634 55.116981) (end 89.126 55.624981) (width 1.5) (layer "F.Cu") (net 3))
 (segment (start 89.38 28.446981) (end 89.634 28.700981) (width 1.5) (layer "F.Cu") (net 3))
 (segment (start 60.678 40.384981) (end 60.678 28.700981) (width 1.5) (layer "F.Cu") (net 3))
 (segment (start 60.932 28.446981) (end 71.092 28.446981) (width 1.5) (layer "F.Cu") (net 3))
 (segment (start 61.04512 40.752101) (end 60.678 40.384981) (width 1.5) (layer "F.Cu") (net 3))
 (segment (start 89.634 28.700981) (end 89.634 55.116981) (width 1.5) (layer "F.Cu") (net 3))
 (segment (start 60.678 28.700981) (end 60.932 28.446981) (width 1.5) (layer "F.Cu") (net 3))
 (segment (start 63.70086 40.752101) (end 61.04512 40.752101) (width 1.5) (layer "F.Cu") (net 3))
 (segment (start 89.126 55.624981) (end 82.12702 55.624981) (width 1.5) (layer "F.Cu") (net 3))
 (segment (start 63.70086 50.912101) (end 51.182101 50.912101) (width 1.5) (layer "F.Cu") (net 15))
 (segment (start 68.2522 50.912101) (end 68.298 50.957901) (width 1.5) (layer "F.Cu") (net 15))
 (segment (start 68.298 50.957901) (end 72.9865 50.957901) (width 1.5) (layer "F.Cu") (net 15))
 (segment (start 72.9865 50.957901) (end 72.9992 50.945201) (width 1.5) (layer "F.Cu") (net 15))
 (segment (start 51.182101 50.912101) (end 51.16 50.89) (width 1.5) (layer "F.Cu") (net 15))
 (segment (start 63.70086 50.912101) (end 68.2522 50.912101) (width 1.5) (layer "F.Cu") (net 15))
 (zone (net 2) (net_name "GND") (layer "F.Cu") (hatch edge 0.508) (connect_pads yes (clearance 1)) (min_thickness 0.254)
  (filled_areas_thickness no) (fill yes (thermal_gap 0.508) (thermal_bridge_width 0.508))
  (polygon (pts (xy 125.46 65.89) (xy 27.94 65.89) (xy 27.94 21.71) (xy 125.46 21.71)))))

